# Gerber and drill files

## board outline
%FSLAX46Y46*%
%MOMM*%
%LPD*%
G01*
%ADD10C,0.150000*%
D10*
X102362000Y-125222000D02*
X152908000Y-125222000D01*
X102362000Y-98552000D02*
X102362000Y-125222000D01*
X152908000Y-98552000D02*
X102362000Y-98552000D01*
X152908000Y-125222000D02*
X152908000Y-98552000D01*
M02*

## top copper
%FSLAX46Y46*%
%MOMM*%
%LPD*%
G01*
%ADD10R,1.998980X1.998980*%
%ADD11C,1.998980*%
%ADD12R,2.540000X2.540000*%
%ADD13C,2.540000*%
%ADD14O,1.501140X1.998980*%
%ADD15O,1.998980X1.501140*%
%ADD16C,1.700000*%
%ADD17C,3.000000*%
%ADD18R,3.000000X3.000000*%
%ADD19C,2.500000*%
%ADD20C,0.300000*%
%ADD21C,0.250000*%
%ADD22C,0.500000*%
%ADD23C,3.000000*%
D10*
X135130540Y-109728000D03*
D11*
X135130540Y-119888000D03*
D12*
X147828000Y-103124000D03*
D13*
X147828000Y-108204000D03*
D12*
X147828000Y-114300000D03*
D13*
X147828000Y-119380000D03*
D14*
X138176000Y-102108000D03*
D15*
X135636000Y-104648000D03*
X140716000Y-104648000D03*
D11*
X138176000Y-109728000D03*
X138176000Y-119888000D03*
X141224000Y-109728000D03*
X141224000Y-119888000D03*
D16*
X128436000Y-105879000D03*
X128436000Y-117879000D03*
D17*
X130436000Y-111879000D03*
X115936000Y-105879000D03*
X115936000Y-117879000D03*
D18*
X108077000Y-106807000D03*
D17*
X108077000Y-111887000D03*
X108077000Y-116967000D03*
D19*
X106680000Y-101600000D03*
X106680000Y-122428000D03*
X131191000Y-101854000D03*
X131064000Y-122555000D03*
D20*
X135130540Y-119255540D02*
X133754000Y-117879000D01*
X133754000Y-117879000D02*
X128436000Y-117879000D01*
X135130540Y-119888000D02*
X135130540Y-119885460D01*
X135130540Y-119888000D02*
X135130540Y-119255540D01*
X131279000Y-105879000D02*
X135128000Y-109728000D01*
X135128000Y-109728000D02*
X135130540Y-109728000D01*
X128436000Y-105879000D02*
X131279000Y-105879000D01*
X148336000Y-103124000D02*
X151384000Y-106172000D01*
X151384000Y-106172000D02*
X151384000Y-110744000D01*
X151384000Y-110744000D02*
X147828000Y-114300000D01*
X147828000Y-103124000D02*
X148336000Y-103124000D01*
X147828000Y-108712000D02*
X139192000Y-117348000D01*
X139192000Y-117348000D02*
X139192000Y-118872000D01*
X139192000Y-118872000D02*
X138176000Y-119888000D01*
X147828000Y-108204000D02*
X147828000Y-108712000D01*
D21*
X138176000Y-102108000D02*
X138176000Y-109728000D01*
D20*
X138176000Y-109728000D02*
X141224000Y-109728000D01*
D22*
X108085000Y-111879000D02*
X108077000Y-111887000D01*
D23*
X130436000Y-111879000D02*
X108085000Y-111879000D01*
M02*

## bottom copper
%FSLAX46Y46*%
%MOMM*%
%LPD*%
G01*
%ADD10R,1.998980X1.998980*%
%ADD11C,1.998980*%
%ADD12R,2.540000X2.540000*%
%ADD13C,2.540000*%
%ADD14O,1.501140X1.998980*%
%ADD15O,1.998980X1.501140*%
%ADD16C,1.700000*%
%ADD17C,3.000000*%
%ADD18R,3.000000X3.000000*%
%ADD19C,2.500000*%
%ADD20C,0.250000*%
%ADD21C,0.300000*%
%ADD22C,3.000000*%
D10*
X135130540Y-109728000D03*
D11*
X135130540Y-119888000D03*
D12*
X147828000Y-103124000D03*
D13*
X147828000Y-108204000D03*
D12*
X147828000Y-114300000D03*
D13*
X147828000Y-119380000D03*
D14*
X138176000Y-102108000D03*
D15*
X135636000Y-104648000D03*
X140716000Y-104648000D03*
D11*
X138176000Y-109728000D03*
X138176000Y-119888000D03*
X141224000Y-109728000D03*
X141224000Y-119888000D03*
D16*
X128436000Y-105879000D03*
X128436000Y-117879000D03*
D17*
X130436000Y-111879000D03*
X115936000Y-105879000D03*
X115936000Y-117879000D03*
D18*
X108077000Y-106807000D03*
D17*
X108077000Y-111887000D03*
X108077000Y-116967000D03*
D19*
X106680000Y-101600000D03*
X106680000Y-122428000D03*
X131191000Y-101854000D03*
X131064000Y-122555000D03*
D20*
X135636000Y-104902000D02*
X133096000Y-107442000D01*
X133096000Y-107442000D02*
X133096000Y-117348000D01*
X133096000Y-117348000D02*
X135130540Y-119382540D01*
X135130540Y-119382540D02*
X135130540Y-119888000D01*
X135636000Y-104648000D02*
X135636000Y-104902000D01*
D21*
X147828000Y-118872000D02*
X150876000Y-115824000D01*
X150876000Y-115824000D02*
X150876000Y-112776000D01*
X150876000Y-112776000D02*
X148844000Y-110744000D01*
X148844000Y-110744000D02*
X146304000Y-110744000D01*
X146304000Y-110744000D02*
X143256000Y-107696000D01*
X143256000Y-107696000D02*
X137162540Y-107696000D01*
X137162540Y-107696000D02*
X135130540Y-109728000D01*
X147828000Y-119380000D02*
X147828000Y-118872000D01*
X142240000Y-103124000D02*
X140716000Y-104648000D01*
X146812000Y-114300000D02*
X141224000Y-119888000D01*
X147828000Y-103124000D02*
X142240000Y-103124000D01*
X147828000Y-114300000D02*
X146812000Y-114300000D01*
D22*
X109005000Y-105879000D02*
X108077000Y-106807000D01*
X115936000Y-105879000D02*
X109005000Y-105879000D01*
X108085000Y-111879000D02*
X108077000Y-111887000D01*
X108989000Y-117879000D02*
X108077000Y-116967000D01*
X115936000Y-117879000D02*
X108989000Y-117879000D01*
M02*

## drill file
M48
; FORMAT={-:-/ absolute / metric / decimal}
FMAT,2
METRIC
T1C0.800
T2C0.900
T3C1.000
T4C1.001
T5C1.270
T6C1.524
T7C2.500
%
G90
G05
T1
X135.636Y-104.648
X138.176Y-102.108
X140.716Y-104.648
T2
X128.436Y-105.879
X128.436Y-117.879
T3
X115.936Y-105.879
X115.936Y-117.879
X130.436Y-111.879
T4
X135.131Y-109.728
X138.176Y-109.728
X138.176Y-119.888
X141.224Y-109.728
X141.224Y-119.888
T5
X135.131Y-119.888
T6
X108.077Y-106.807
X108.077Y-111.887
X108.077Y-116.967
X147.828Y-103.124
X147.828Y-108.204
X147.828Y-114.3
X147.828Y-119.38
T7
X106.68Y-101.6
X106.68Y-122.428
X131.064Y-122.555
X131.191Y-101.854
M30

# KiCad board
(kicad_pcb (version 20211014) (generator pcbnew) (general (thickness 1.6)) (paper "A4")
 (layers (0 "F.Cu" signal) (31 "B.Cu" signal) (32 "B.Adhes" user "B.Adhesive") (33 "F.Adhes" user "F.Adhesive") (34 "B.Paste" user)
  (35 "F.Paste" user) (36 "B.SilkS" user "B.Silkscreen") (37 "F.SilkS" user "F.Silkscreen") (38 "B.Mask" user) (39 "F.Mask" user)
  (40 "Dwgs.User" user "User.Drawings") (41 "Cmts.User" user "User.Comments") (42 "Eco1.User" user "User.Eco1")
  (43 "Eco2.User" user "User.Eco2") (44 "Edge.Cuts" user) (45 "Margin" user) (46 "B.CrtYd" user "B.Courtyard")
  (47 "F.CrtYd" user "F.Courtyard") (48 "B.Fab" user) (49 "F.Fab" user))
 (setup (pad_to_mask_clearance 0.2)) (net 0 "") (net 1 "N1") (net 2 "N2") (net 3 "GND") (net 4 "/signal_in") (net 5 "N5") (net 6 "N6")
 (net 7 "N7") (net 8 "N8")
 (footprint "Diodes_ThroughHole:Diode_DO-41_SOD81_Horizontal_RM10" (layer "F.Cu") (at 135.128 109.728 -90)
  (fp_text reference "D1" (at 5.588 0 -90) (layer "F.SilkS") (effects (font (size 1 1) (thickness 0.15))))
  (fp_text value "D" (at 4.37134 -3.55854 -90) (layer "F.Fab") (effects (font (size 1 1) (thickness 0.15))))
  (pad "1" thru_hole rect locked (at 0 -0.00254 90) (size 1.99898 1.99898) (drill 1.00076) (layers *.Cu *.Mask "F.SilkS") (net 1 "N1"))
  (pad "2" thru_hole circle locked (at 10.16 -0.00254 90) (size 1.99898 1.99898) (drill 1.27) (layers *.Cu *.Mask "F.SilkS") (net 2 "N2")))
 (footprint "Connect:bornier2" (layer "F.Cu") (at 147.828 105.664 -90)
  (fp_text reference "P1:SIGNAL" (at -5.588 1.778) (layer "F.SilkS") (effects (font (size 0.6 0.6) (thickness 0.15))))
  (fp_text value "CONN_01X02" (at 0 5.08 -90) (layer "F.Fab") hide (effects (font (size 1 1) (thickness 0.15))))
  (pad "1" thru_hole rect locked (at -2.54 0 270) (size 2.54 2.54) (drill 1.524) (layers *.Cu *.Mask "F.SilkS") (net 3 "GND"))
  (pad "2" thru_hole circle locked (at 2.54 0 270) (size 2.54 2.54) (drill 1.524) (layers *.Cu *.Mask "F.SilkS") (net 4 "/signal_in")))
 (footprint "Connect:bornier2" (layer "F.Cu") (at 147.828 116.84 -90)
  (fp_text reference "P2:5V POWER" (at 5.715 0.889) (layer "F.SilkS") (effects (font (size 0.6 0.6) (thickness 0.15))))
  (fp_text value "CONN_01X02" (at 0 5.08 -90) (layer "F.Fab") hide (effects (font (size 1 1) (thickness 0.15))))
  (pad "1" thru_hole rect locked (at -2.54 0 270) (size 2.54 2.54) (drill 1.524) (layers *.Cu *.Mask "F.SilkS") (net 3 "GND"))
  (pad "2" thru_hole circle locked (at 2.54 0 270) (size 2.54 2.54) (drill 1.524) (layers *.Cu *.Mask "F.SilkS") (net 1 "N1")))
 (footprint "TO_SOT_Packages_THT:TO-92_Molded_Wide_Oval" (layer "F.Cu") (at 135.636 104.648)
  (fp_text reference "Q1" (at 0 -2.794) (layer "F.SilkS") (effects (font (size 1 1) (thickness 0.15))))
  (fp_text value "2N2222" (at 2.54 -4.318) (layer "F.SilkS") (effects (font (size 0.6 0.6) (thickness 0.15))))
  (pad "1" thru_hole oval locked (at 2.54 -2.54 90) (size 1.99898 1.50114) (drill 0.8) (layers *.Cu *.Mask "F.SilkS") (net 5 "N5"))
  (pad "2" thru_hole oval locked (at 0 0 90) (size 1.50114 1.99898) (drill 0.8) (layers *.Cu *.Mask "F.SilkS") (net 2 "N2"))
  (pad "3" thru_hole oval locked (at 5.08 0 90) (size 1.50114 1.99898) (drill 0.8) (layers *.Cu *.Mask "F.SilkS") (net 3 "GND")))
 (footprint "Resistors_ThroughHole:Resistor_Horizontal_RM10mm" (layer "F.Cu") (at 138.176 114.808 -90)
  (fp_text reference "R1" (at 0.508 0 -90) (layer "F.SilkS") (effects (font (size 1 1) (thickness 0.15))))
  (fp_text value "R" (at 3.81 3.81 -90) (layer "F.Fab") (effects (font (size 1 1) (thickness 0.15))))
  (pad "1" thru_hole circle locked (at -5.08 0 270) (size 1.99898 1.99898) (drill 1.00076) (layers *.Cu *.SilkS *.Mask) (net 5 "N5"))
  (pad "2" thru_hole circle locked (at 5.08 0 270) (size 1.99898 1.99898) (drill 1.00076) (layers *.Cu *.SilkS *.Mask) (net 4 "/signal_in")))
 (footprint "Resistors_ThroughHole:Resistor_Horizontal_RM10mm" (layer "F.Cu") (at 141.224 114.808 -90)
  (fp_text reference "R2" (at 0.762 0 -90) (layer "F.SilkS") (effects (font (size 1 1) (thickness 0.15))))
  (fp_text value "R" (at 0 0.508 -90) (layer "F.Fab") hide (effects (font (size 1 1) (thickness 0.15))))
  (pad "1" thru_hole circle locked (at -5.08 0 270) (size 1.99898 1.99898) (drill 1.00076) (layers *.Cu *.SilkS *.Mask) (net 5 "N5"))
  (pad "2" thru_hole circle locked (at 5.08 0 270) (size 1.99898 1.99898) (drill 1.00076) (layers *.Cu *.SilkS *.Mask) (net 3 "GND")))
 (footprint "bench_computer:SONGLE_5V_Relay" (layer "F.Cu") (at 122.936 111.379)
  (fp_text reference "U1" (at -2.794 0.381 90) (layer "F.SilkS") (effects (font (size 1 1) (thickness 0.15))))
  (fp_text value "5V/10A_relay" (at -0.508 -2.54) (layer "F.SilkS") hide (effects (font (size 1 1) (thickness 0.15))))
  (pad "1" thru_hole circle locked (at 5.5 -5.5) (size 1.7 1.7) (drill 0.9) (layers *.Cu *.Mask "F.SilkS") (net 1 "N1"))
  (pad "2" thru_hole circle locked (at 5.5 6.5) (size 1.7 1.7) (drill 0.9) (layers *.Cu *.Mask "F.SilkS") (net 2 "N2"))
  (pad "3" thru_hole circle locked (at 7.5 0.5) (size 3 3) (drill 1) (layers *.Cu *.Mask "F.SilkS") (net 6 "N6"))
  (pad "4" thru_hole circle locked (at -7 -5.5) (size 3 3) (drill 1) (layers *.Cu *.Mask "F.SilkS") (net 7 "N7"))
  (pad "5" thru_hole circle locked (at -7 6.5) (size 3 3) (drill 1) (layers *.Cu *.Mask "F.SilkS") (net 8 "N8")))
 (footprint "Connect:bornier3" (layer "F.Cu") (at 108.077 111.887 -90)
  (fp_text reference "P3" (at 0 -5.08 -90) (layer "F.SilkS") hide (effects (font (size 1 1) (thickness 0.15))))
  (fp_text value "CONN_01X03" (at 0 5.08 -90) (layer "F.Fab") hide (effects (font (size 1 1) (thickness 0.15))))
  (pad "1" thru_hole rect locked (at -5.08 0 270) (size 3 3) (drill 1.524) (layers *.Cu *.Mask "F.SilkS") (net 7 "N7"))
  (pad "2" thru_hole circle locked (at 0 0 270) (size 3 3) (drill 1.524) (layers *.Cu *.Mask "F.SilkS") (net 6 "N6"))
  (pad "3" thru_hole circle locked (at 5.08 0 270) (size 3 3) (drill 1.524) (layers *.Cu *.Mask "F.SilkS") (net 8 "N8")))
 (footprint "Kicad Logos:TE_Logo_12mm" (layer "F.Cu") (at 118.364 101.219)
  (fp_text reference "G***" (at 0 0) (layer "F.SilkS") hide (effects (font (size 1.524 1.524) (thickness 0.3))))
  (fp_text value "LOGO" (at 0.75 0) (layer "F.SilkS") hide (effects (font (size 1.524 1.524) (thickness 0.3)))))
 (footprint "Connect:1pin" (layer "F.Cu") (at 106.68 101.6)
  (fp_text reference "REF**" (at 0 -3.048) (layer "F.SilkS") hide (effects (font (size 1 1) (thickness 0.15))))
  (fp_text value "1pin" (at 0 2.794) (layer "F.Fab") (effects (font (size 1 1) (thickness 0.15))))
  (pad "1" thru_hole circle locked (at 0 0) (size 2.5 2.5) (drill 2.5) (layers *.Cu *.Mask)))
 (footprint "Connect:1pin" (layer "F.Cu") (at 106.68 122.428)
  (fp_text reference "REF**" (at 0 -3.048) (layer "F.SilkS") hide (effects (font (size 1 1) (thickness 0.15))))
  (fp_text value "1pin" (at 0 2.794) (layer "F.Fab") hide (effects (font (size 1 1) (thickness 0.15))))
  (pad "1" thru_hole circle locked (at 0 0) (size 2.5 2.5) (drill 2.5) (layers *.Cu *.Mask)))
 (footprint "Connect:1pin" (layer "F.Cu") (at 131.191 101.854)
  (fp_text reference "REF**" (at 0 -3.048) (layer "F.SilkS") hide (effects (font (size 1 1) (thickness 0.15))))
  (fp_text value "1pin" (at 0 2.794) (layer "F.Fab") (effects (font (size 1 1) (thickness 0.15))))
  (pad "1" thru_hole circle locked (at 0 0) (size 2.5 2.5) (drill 2.5) (layers *.Cu *.Mask)))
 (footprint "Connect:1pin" (layer "F.Cu") (at 131.064 122.555)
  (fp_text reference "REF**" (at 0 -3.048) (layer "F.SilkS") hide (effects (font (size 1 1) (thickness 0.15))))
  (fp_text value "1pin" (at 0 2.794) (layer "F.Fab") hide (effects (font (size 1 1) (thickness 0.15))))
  (pad "1" thru_hole circle locked (at 0 0) (size 2.5 2.5) (drill 2.5) (layers *.Cu *.Mask)))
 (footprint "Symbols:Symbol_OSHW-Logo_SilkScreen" (layer "B.Cu") (at 122.428 111.125 180)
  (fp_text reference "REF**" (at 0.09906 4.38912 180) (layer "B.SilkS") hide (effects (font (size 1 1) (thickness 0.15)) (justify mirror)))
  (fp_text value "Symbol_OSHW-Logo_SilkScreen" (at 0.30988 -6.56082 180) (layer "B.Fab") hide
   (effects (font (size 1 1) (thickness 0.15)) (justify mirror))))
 (gr_line (start 102.362 125.222) (end 152.908 125.222) (layer "Edge.Cuts") (width 0.15))
 (gr_line (start 102.362 98.552) (end 102.362 125.222) (layer "Edge.Cuts") (width 0.15))
 (gr_line (start 152.908 98.552) (end 102.362 98.552) (layer "Edge.Cuts") (width 0.15))
 (gr_line (start 152.908 125.222) (end 152.908 98.552) (layer "Edge.Cuts") (width 0.15))
 (segment (start 135.13054 119.25554) (end 133.754 117.879) (width 0.3) (layer "F.Cu") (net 2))
 (segment (start 133.754 117.879) (end 128.436 117.879) (width 0.3) (layer "F.Cu") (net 2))
 (segment (start 135.13054 119.888) (end 135.13054 119.88546) (width 0.3) (layer "F.Cu") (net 2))
 (segment (start 135.13054 119.888) (end 135.13054 119.25554) (width 0.3) (layer "F.Cu") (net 2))
 (segment (start 135.636 104.902) (end 133.096 107.442) (width 0.25) (layer "B.Cu") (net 2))
 (segment (start 133.096 107.442) (end 133.096 117.348) (width 0.25) (layer "B.Cu") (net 2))
 (segment (start 133.096 117.348) (end 135.13054 119.38254) (width 0.25) (layer "B.Cu") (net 2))
 (segment (start 135.13054 119.38254) (end 135.13054 119.888) (width 0.25) (layer "B.Cu") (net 2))
 (segment (start 135.636 104.648) (end 135.636 104.902) (width 0.25) (layer "B.Cu") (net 2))
 (segment (start 131.279 105.879) (end 135.128 109.728) (width 0.3) (layer "F.Cu") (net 1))
 (segment (start 135.128 109.728) (end 135.13054 109.728) (width 0.3) (layer "F.Cu") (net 1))
 (segment (start 128.436 105.879) (end 131.279 105.879) (width 0.3) (layer "F.Cu") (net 1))
 (segment (start 147.828 118.872) (end 150.876 115.824) (width 0.3) (layer "B.Cu") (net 1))
 (segment (start 150.876 115.824) (end 150.876 112.776) (width 0.3) (layer "B.Cu") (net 1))
 (segment (start 150.876 112.776) (end 148.844 110.744) (width 0.3) (layer "B.Cu") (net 1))
 (segment (start 148.844 110.744) (end 146.304 110.744) (width 0.3) (layer "B.Cu") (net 1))
 (segment (start 146.304 110.744) (end 143.256 107.696) (width 0.3) (layer "B.Cu") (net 1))
 (segment (start 143.256 107.696) (end 137.16254 107.696) (width 0.3) (layer "B.Cu") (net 1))
 (segment (start 137.16254 107.696) (end 135.13054 109.728) (width 0.3) (layer "B.Cu") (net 1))
 (segment (start 147.828 119.38) (end 147.828 118.872) (width 0.3) (layer "B.Cu") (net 1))
 (segment (start 148.336 103.124) (end 151.384 106.172) (width 0.3) (layer "F.Cu") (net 3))
 (segment (start 151.384 106.172) (end 151.384 110.744) (width 0.3) (layer "F.Cu") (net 3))
 (segment (start 151.384 110.744) (end 147.828 114.3) (width 0.3) (layer "F.Cu") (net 3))
 (segment (start 147.828 103.124) (end 148.336 103.124) (width 0.3) (layer "F.Cu") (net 3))
 (segment (start 142.24 103.124) (end 140.716 104.648) (width 0.3) (layer "B.Cu") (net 3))
 (segment (start 146.812 114.3) (end 141.224 119.888) (width 0.3) (layer "B.Cu") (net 3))
 (segment (start 147.828 103.124) (end 142.24 103.124) (width 0.3) (layer "B.Cu") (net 3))
 (segment (start 147.828 114.3) (end 146.812 114.3) (width 0.3) (layer "B.Cu") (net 3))
 (segment (start 147.828 108.712) (end 139.192 117.348) (width 0.3) (layer "F.Cu") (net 4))
 (segment (start 139.192 117.348) (end 139.192 118.872) (width 0.3) (layer "F.Cu") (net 4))
 (segment (start 139.192 118.872) (end 138.176 119.888) (width 0.3) (layer "F.Cu") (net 4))
 (segment (start 147.828 108.204) (end 147.828 108.712) (width 0.3) (layer "F.Cu") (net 4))
 (segment (start 138.176 102.108) (end 138.176 109.728) (width 0.25) (layer "F.Cu") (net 5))
 (segment (start 138.176 109.728) (end 141.224 109.728) (width 0.3) (layer "F.Cu") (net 5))
 (segment (start 109.005 105.879) (end 108.077 106.807) (width 3) (layer "B.Cu") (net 7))
 (segment (start 115.936 105.879) (end 109.005 105.879) (width 3) (layer "B.Cu") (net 7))
 (segment (start 108.085 111.879) (end 108.077 111.887) (width 0.5) (layer "F.Cu") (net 6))
 (segment (start 130.436 111.879) (end 108.085 111.879) (width 3) (layer "F.Cu") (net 6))
 (segment (start 108.085 111.879) (end 108.077 111.887) (width 3) (layer "B.Cu") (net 6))
 (segment (start 108.989 117.879) (end 108.077 116.967) (width 3) (layer "B.Cu") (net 8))
 (segment (start 115.936 117.879) (end 108.989 117.879) (width 3) (layer "B.Cu") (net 8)))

